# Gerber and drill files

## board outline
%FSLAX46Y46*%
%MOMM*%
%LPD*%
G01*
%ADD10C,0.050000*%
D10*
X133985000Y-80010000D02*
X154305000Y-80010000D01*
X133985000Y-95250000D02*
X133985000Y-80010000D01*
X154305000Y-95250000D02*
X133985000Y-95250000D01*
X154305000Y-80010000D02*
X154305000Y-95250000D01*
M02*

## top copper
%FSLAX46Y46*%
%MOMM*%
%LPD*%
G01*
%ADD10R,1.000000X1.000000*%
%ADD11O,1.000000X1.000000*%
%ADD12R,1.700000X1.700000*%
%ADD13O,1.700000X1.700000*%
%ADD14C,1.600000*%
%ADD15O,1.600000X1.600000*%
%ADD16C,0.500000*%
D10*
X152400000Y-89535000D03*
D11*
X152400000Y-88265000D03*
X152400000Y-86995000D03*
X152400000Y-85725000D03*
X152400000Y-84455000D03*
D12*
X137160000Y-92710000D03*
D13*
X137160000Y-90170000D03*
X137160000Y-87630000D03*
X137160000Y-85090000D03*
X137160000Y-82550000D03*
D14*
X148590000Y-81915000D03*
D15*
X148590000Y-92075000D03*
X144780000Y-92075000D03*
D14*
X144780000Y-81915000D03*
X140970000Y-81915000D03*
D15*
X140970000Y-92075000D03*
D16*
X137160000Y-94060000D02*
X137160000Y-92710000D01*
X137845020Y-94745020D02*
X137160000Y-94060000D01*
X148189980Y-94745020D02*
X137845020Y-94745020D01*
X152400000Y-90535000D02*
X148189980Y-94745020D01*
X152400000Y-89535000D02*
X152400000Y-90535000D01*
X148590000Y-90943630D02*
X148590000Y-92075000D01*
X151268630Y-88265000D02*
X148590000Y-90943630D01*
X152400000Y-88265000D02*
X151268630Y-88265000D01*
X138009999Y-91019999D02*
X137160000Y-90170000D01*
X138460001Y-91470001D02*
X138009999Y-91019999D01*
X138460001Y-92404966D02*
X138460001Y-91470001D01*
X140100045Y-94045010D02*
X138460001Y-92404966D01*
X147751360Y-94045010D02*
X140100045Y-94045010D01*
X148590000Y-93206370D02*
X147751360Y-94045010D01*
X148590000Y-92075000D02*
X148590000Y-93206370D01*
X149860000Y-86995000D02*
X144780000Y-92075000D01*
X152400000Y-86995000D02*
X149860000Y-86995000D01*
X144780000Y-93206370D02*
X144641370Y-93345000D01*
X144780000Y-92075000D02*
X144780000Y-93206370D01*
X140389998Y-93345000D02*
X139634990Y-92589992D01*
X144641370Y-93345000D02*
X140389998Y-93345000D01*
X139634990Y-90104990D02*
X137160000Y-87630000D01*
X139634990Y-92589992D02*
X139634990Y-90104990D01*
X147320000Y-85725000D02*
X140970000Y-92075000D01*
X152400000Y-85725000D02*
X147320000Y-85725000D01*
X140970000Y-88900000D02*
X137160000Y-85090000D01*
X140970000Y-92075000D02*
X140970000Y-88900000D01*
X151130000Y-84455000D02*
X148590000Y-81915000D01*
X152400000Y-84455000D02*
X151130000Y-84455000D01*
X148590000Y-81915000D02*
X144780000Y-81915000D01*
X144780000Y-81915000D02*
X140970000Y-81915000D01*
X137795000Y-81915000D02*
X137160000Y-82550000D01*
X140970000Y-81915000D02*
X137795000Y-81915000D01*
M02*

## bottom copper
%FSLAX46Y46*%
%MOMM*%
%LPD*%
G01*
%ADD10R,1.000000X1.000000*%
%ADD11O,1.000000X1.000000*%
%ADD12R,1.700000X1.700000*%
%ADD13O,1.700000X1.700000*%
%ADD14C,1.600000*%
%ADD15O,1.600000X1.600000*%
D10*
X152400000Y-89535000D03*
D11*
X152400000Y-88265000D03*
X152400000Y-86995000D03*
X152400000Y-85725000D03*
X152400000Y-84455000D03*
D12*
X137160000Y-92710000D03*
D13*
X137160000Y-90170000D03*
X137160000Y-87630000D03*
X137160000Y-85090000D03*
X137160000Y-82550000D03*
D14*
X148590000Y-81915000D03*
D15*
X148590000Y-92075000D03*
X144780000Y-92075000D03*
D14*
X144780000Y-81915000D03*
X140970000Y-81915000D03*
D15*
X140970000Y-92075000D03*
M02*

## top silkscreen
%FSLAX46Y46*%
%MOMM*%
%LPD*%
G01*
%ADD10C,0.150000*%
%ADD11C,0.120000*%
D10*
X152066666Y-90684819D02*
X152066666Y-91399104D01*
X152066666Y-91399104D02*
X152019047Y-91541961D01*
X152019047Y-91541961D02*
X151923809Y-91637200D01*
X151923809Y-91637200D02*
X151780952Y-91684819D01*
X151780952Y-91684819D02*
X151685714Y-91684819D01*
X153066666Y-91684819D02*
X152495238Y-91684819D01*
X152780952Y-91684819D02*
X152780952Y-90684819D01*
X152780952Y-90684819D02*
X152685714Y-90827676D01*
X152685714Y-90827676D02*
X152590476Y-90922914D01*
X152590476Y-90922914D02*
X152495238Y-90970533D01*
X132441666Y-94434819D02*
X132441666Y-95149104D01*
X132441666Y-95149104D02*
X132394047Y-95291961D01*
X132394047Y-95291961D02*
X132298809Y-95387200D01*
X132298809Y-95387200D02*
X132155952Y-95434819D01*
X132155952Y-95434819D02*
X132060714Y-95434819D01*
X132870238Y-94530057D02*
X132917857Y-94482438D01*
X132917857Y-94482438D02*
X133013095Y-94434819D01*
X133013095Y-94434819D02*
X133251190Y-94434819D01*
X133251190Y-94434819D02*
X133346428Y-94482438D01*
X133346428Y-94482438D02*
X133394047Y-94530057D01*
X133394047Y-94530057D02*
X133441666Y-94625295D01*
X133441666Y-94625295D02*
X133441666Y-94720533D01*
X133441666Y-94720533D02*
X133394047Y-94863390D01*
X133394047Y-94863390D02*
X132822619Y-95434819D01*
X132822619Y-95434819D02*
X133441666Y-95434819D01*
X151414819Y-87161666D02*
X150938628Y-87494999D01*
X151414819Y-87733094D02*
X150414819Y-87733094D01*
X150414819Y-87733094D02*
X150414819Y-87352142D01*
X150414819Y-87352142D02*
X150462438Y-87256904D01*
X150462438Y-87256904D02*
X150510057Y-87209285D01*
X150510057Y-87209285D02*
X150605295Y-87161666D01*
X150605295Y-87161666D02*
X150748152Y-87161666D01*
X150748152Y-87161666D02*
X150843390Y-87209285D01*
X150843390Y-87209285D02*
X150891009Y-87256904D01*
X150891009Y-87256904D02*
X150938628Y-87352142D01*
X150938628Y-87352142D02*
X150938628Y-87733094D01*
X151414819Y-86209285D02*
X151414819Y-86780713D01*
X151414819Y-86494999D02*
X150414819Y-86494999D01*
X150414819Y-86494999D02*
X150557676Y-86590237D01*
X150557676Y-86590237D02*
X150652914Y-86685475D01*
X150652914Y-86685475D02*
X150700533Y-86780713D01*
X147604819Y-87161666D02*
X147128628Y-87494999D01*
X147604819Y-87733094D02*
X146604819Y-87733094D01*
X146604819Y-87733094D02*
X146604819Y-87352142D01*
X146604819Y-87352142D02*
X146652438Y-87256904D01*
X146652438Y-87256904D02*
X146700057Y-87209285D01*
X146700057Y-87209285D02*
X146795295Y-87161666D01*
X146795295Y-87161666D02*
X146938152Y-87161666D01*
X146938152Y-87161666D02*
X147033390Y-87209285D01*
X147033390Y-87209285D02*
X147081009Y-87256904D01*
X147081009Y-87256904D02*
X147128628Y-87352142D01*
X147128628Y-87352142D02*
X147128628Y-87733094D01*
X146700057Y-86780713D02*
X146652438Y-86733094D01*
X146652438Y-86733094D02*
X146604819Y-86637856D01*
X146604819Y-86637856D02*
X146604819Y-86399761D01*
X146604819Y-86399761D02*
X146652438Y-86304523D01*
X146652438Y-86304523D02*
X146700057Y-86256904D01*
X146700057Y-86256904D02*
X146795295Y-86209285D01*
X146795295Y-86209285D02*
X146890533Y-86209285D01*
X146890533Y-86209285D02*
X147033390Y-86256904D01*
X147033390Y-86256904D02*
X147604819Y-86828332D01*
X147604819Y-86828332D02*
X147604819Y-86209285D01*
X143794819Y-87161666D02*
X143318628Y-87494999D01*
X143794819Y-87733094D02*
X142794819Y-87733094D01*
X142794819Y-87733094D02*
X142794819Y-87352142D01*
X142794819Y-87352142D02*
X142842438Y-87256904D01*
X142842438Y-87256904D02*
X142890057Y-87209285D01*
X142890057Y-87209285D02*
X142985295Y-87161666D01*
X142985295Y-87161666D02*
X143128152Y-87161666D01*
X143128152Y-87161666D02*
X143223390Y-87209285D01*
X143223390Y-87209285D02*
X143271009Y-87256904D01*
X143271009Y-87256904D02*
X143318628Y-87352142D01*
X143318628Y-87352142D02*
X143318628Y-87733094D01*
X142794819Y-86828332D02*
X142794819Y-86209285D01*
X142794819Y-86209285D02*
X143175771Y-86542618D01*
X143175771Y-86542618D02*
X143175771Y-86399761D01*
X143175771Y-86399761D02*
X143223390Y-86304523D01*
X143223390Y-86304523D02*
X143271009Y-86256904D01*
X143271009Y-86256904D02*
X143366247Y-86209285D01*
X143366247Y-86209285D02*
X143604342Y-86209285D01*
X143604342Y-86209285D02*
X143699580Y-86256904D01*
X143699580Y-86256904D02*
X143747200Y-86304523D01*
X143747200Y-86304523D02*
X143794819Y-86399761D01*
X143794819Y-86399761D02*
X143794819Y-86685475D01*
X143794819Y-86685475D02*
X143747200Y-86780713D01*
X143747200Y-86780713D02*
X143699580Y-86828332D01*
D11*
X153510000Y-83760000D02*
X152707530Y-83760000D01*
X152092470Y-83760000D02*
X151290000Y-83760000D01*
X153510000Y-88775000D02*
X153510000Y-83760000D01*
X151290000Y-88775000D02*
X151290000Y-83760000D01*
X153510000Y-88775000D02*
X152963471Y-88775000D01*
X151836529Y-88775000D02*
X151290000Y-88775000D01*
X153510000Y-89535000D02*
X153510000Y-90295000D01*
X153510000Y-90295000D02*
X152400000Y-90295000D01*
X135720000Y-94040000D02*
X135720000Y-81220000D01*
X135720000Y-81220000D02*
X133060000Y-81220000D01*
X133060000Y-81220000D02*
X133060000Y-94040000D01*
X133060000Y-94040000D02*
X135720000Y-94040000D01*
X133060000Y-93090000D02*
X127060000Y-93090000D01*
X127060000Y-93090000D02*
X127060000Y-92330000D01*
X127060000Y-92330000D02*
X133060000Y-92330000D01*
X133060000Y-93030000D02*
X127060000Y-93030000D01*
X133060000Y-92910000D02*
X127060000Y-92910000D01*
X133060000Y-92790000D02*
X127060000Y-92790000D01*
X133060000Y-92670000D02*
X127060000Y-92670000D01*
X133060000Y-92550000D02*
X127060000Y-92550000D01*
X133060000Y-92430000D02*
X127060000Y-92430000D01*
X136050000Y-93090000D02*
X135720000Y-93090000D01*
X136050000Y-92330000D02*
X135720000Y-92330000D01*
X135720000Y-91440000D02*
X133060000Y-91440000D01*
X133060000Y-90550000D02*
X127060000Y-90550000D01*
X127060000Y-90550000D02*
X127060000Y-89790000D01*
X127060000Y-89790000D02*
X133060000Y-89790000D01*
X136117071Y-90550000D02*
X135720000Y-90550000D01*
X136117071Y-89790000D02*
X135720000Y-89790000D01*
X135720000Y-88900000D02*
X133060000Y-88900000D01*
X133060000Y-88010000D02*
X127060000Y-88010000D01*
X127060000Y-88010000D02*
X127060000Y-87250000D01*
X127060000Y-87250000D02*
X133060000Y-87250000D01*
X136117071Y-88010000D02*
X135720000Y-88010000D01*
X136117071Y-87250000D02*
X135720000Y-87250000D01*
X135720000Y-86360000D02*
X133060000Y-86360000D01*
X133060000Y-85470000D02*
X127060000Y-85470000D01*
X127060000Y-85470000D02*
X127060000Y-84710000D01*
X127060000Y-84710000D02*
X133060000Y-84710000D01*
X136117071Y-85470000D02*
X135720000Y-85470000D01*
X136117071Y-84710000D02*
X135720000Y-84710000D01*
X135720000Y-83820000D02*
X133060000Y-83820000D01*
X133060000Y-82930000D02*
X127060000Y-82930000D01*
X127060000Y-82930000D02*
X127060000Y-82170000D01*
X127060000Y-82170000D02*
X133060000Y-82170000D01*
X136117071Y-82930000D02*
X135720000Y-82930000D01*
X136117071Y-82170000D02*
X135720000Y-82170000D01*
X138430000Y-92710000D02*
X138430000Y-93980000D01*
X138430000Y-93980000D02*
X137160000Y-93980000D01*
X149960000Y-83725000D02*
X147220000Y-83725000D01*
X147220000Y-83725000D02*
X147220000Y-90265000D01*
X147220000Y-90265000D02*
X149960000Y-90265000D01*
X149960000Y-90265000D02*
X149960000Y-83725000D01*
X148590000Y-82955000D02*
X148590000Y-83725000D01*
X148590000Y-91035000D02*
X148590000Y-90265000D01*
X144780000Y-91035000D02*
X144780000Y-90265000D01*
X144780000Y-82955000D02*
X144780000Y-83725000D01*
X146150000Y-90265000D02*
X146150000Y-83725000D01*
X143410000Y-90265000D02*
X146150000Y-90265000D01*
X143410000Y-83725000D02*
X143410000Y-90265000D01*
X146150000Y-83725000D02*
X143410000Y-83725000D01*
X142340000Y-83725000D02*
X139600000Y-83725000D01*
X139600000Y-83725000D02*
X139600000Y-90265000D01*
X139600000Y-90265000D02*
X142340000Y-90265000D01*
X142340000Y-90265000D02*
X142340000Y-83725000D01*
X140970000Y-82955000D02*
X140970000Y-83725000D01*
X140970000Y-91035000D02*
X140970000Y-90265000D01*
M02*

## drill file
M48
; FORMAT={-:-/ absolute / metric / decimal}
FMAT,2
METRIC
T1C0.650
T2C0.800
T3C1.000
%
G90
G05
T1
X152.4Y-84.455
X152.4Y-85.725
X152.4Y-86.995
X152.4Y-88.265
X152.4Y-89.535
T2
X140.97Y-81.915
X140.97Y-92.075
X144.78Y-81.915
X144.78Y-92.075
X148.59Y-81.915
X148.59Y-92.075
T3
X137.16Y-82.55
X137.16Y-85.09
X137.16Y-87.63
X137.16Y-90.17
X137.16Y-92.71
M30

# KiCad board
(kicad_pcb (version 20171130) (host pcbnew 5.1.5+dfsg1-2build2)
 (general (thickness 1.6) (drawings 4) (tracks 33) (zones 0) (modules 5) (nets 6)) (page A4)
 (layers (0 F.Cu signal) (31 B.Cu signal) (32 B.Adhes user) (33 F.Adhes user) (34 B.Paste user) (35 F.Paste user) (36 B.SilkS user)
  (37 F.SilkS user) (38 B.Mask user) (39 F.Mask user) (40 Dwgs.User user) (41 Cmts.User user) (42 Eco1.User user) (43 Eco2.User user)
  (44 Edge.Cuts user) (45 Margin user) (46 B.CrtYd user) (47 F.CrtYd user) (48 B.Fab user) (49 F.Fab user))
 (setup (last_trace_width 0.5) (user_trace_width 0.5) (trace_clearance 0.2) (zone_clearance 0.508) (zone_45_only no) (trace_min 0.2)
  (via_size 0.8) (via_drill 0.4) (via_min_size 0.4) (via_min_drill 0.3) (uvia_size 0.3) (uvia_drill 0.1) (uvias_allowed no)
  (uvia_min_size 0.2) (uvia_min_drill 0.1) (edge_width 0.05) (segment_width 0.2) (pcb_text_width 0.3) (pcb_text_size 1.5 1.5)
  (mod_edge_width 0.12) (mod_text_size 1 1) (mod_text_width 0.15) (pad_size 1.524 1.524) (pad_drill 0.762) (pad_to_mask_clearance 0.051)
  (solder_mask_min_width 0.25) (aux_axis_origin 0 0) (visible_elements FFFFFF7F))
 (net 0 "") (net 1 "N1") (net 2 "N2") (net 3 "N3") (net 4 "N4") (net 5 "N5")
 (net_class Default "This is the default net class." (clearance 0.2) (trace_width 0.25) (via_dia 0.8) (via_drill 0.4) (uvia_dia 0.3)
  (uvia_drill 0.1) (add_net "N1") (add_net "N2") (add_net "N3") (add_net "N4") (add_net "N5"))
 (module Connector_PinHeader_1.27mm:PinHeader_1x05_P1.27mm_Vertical (layer F.Cu) (at 152.4 89.535 180)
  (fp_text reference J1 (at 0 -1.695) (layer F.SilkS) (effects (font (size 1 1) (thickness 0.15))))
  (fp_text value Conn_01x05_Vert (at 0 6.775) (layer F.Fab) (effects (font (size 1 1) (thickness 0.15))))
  (fp_line (start -1.11 5.775) (end -0.30753 5.775) (layer F.SilkS) (width 0.12))
  (fp_line (start 0.30753 5.775) (end 1.11 5.775) (layer F.SilkS) (width 0.12))
  (fp_line (start -1.11 0.76) (end -1.11 5.775) (layer F.SilkS) (width 0.12))
  (fp_line (start 1.11 0.76) (end 1.11 5.775) (layer F.SilkS) (width 0.12))
  (fp_line (start -1.11 0.76) (end -0.563471 0.76) (layer F.SilkS) (width 0.12))
  (fp_line (start 0.563471 0.76) (end 1.11 0.76) (layer F.SilkS) (width 0.12))
  (fp_line (start -1.11 0) (end -1.11 -0.76) (layer F.SilkS) (width 0.12))
  (fp_line (start -1.11 -0.76) (end 0 -0.76) (layer F.SilkS) (width 0.12))
  (pad 1 thru_hole rect (at 0 0 180) (size 1 1) (drill 0.65) (layers *.Cu *.Mask) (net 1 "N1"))
  (pad 2 thru_hole oval (at 0 1.27 180) (size 1 1) (drill 0.65) (layers *.Cu *.Mask) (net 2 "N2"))
  (pad 3 thru_hole oval (at 0 2.54 180) (size 1 1) (drill 0.65) (layers *.Cu *.Mask) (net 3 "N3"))
  (pad 4 thru_hole oval (at 0 3.81 180) (size 1 1) (drill 0.65) (layers *.Cu *.Mask) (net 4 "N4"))
  (pad 5 thru_hole oval (at 0 5.08 180) (size 1 1) (drill 0.65) (layers *.Cu *.Mask) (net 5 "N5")))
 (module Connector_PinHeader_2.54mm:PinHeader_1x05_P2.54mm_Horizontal (layer F.Cu) (at 137.16 92.71 180)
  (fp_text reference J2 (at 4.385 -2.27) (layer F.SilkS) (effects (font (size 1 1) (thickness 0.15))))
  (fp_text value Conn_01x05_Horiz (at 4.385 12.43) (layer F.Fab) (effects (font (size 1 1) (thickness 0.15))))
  (fp_line (start 1.44 -1.33) (end 1.44 11.49) (layer F.SilkS) (width 0.12))
  (fp_line (start 1.44 11.49) (end 4.1 11.49) (layer F.SilkS) (width 0.12))
  (fp_line (start 4.1 11.49) (end 4.1 -1.33) (layer F.SilkS) (width 0.12))
  (fp_line (start 4.1 -1.33) (end 1.44 -1.33) (layer F.SilkS) (width 0.12))
  (fp_line (start 4.1 -0.38) (end 10.1 -0.38) (layer F.SilkS) (width 0.12))
  (fp_line (start 10.1 -0.38) (end 10.1 0.38) (layer F.SilkS) (width 0.12))
  (fp_line (start 10.1 0.38) (end 4.1 0.38) (layer F.SilkS) (width 0.12))
  (fp_line (start 4.1 -0.32) (end 10.1 -0.32) (layer F.SilkS) (width 0.12))
  (fp_line (start 4.1 -0.2) (end 10.1 -0.2) (layer F.SilkS) (width 0.12))
  (fp_line (start 4.1 -0.08) (end 10.1 -0.08) (layer F.SilkS) (width 0.12))
  (fp_line (start 4.1 0.04) (end 10.1 0.04) (layer F.SilkS) (width 0.12))
  (fp_line (start 4.1 0.16) (end 10.1 0.16) (layer F.SilkS) (width 0.12))
  (fp_line (start 4.1 0.28) (end 10.1 0.28) (layer F.SilkS) (width 0.12))
  (fp_line (start 1.11 -0.38) (end 1.44 -0.38) (layer F.SilkS) (width 0.12))
  (fp_line (start 1.11 0.38) (end 1.44 0.38) (layer F.SilkS) (width 0.12))
  (fp_line (start 1.44 1.27) (end 4.1 1.27) (layer F.SilkS) (width 0.12))
  (fp_line (start 4.1 2.16) (end 10.1 2.16) (layer F.SilkS) (width 0.12))
  (fp_line (start 10.1 2.16) (end 10.1 2.92) (layer F.SilkS) (width 0.12))
  (fp_line (start 10.1 2.92) (end 4.1 2.92) (layer F.SilkS) (width 0.12))
  (fp_line (start 1.042929 2.16) (end 1.44 2.16) (layer F.SilkS) (width 0.12))
  (fp_line (start 1.042929 2.92) (end 1.44 2.92) (layer F.SilkS) (width 0.12))
  (fp_line (start 1.44 3.81) (end 4.1 3.81) (layer F.SilkS) (width 0.12))
  (fp_line (start 4.1 4.7) (end 10.1 4.7) (layer F.SilkS) (width 0.12))
  (fp_line (start 10.1 4.7) (end 10.1 5.46) (layer F.SilkS) (width 0.12))
  (fp_line (start 10.1 5.46) (end 4.1 5.46) (layer F.SilkS) (width 0.12))
  (fp_line (start 1.042929 4.7) (end 1.44 4.7) (layer F.SilkS) (width 0.12))
  (fp_line (start 1.042929 5.46) (end 1.44 5.46) (layer F.SilkS) (width 0.12))
  (fp_line (start 1.44 6.35) (end 4.1 6.35) (layer F.SilkS) (width 0.12))
  (fp_line (start 4.1 7.24) (end 10.1 7.24) (layer F.SilkS) (width 0.12))
  (fp_line (start 10.1 7.24) (end 10.1 8) (layer F.SilkS) (width 0.12))
  (fp_line (start 10.1 8) (end 4.1 8) (layer F.SilkS) (width 0.12))
  (fp_line (start 1.042929 7.24) (end 1.44 7.24) (layer F.SilkS) (width 0.12))
  (fp_line (start 1.042929 8) (end 1.44 8) (layer F.SilkS) (width 0.12))
  (fp_line (start 1.44 8.89) (end 4.1 8.89) (layer F.SilkS) (width 0.12))
  (fp_line (start 4.1 9.78) (end 10.1 9.78) (layer F.SilkS) (width 0.12))
  (fp_line (start 10.1 9.78) (end 10.1 10.54) (layer F.SilkS) (width 0.12))
  (fp_line (start 10.1 10.54) (end 4.1 10.54) (layer F.SilkS) (width 0.12))
  (fp_line (start 1.042929 9.78) (end 1.44 9.78) (layer F.SilkS) (width 0.12))
  (fp_line (start 1.042929 10.54) (end 1.44 10.54) (layer F.SilkS) (width 0.12))
  (fp_line (start -1.27 0) (end -1.27 -1.27) (layer F.SilkS) (width 0.12))
  (fp_line (start -1.27 -1.27) (end 0 -1.27) (layer F.SilkS) (width 0.12))
  (pad 1 thru_hole rect (at 0 0 180) (size 1.7 1.7) (drill 1) (layers *.Cu *.Mask) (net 1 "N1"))
  (pad 2 thru_hole oval (at 0 2.54 180) (size 1.7 1.7) (drill 1) (layers *.Cu *.Mask) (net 2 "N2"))
  (pad 3 thru_hole oval (at 0 5.08 180) (size 1.7 1.7) (drill 1) (layers *.Cu *.Mask) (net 3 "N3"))
  (pad 4 thru_hole oval (at 0 7.62 180) (size 1.7 1.7) (drill 1) (layers *.Cu *.Mask) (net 4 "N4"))
  (pad 5 thru_hole oval (at 0 10.16 180) (size 1.7 1.7) (drill 1) (layers *.Cu *.Mask) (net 5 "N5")))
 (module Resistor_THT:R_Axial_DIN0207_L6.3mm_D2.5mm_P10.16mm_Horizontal (layer F.Cu) (at 148.59 81.915 270)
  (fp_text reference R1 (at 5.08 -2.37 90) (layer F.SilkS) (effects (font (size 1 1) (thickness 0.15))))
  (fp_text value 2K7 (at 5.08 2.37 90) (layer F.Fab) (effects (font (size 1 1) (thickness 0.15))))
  (fp_line (start 1.81 -1.37) (end 1.81 1.37) (layer F.SilkS) (width 0.12))
  (fp_line (start 1.81 1.37) (end 8.35 1.37) (layer F.SilkS) (width 0.12))
  (fp_line (start 8.35 1.37) (end 8.35 -1.37) (layer F.SilkS) (width 0.12))
  (fp_line (start 8.35 -1.37) (end 1.81 -1.37) (layer F.SilkS) (width 0.12))
  (fp_line (start 1.04 0) (end 1.81 0) (layer F.SilkS) (width 0.12))
  (fp_line (start 9.12 0) (end 8.35 0) (layer F.SilkS) (width 0.12))
  (pad 1 thru_hole circle (at 0 0 270) (size 1.6 1.6) (drill 0.8) (layers *.Cu *.Mask) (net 5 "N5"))
  (pad 2 thru_hole oval (at 10.16 0 270) (size 1.6 1.6) (drill 0.8) (layers *.Cu *.Mask) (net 2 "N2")))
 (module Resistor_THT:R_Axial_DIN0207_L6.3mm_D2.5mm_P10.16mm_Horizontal (layer F.Cu) (at 144.78 81.915 270)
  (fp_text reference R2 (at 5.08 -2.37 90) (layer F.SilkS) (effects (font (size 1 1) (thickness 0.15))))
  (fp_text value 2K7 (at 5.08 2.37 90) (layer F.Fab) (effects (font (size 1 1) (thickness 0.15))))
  (fp_line (start 9.12 0) (end 8.35 0) (layer F.SilkS) (width 0.12))
  (fp_line (start 1.04 0) (end 1.81 0) (layer F.SilkS) (width 0.12))
  (fp_line (start 8.35 -1.37) (end 1.81 -1.37) (layer F.SilkS) (width 0.12))
  (fp_line (start 8.35 1.37) (end 8.35 -1.37) (layer F.SilkS) (width 0.12))
  (fp_line (start 1.81 1.37) (end 8.35 1.37) (layer F.SilkS) (width 0.12))
  (fp_line (start 1.81 -1.37) (end 1.81 1.37) (layer F.SilkS) (width 0.12))
  (pad 2 thru_hole oval (at 10.16 0 270) (size 1.6 1.6) (drill 0.8) (layers *.Cu *.Mask) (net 3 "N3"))
  (pad 1 thru_hole circle (at 0 0 270) (size 1.6 1.6) (drill 0.8) (layers *.Cu *.Mask) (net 5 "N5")))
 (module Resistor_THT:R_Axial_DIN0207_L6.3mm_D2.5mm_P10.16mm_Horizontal (layer F.Cu) (at 140.97 81.915 270)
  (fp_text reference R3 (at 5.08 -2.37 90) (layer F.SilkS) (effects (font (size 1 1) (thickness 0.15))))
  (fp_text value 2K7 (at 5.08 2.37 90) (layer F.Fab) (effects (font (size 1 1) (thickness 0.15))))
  (fp_line (start 1.81 -1.37) (end 1.81 1.37) (layer F.SilkS) (width 0.12))
  (fp_line (start 1.81 1.37) (end 8.35 1.37) (layer F.SilkS) (width 0.12))
  (fp_line (start 8.35 1.37) (end 8.35 -1.37) (layer F.SilkS) (width 0.12))
  (fp_line (start 8.35 -1.37) (end 1.81 -1.37) (layer F.SilkS) (width 0.12))
  (fp_line (start 1.04 0) (end 1.81 0) (layer F.SilkS) (width 0.12))
  (fp_line (start 9.12 0) (end 8.35 0) (layer F.SilkS) (width 0.12))
  (pad 1 thru_hole circle (at 0 0 270) (size 1.6 1.6) (drill 0.8) (layers *.Cu *.Mask) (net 5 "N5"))
  (pad 2 thru_hole oval (at 10.16 0 270) (size 1.6 1.6) (drill 0.8) (layers *.Cu *.Mask) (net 4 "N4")))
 (gr_line (start 133.985 80.01) (end 154.305 80.01) (layer Edge.Cuts) (width 0.05))
 (gr_line (start 133.985 95.25) (end 133.985 80.01) (layer Edge.Cuts) (width 0.05))
 (gr_line (start 154.305 95.25) (end 133.985 95.25) (layer Edge.Cuts) (width 0.05))
 (gr_line (start 154.305 80.01) (end 154.305 95.25) (layer Edge.Cuts) (width 0.05))
 (segment (start 137.16 94.06) (end 137.16 92.71) (width 0.5) (layer F.Cu) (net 1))
 (segment (start 137.84502 94.74502) (end 137.16 94.06) (width 0.5) (layer F.Cu) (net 1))
 (segment (start 148.18998 94.74502) (end 137.84502 94.74502) (width 0.5) (layer F.Cu) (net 1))
 (segment (start 152.4 90.535) (end 148.18998 94.74502) (width 0.5) (layer F.Cu) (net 1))
 (segment (start 152.4 89.535) (end 152.4 90.535) (width 0.5) (layer F.Cu) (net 1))
 (segment (start 148.59 90.94363) (end 148.59 92.075) (width 0.5) (layer F.Cu) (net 2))
 (segment (start 151.26863 88.265) (end 148.59 90.94363) (width 0.5) (layer F.Cu) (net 2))
 (segment (start 152.4 88.265) (end 151.26863 88.265) (width 0.5) (layer F.Cu) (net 2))
 (segment (start 138.009999 91.019999) (end 137.16 90.17) (width 0.5) (layer F.Cu) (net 2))
 (segment (start 138.460001 91.470001) (end 138.009999 91.019999) (width 0.5) (layer F.Cu) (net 2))
 (segment (start 138.460001 92.404966) (end 138.460001 91.470001) (width 0.5) (layer F.Cu) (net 2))
 (segment (start 140.100045 94.04501) (end 138.460001 92.404966) (width 0.5) (layer F.Cu) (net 2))
 (segment (start 147.75136 94.04501) (end 140.100045 94.04501) (width 0.5) (layer F.Cu) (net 2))
 (segment (start 148.59 93.20637) (end 147.75136 94.04501) (width 0.5) (layer F.Cu) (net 2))
 (segment (start 148.59 92.075) (end 148.59 93.20637) (width 0.5) (layer F.Cu) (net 2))
 (segment (start 149.86 86.995) (end 144.78 92.075) (width 0.5) (layer F.Cu) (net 3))
 (segment (start 152.4 86.995) (end 149.86 86.995) (width 0.5) (layer F.Cu) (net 3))
 (segment (start 144.78 93.20637) (end 144.64137 93.345) (width 0.5) (layer F.Cu) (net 3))
 (segment (start 144.78 92.075) (end 144.78 93.20637) (width 0.5) (layer F.Cu) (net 3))
 (segment (start 140.389998 93.345) (end 139.63499 92.589992) (width 0.5) (layer F.Cu) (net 3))
 (segment (start 144.64137 93.345) (end 140.389998 93.345) (width 0.5) (layer F.Cu) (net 3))
 (segment (start 139.63499 90.10499) (end 137.16 87.63) (width 0.5) (layer F.Cu) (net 3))
 (segment (start 139.63499 92.589992) (end 139.63499 90.10499) (width 0.5) (layer F.Cu) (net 3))
 (segment (start 147.32 85.725) (end 140.97 92.075) (width 0.5) (layer F.Cu) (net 4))
 (segment (start 152.4 85.725) (end 147.32 85.725) (width 0.5) (layer F.Cu) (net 4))
 (segment (start 140.97 88.9) (end 137.16 85.09) (width 0.5) (layer F.Cu) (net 4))
 (segment (start 140.97 92.075) (end 140.97 88.9) (width 0.5) (layer F.Cu) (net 4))
 (segment (start 151.13 84.455) (end 148.59 81.915) (width 0.5) (layer F.Cu) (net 5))
 (segment (start 152.4 84.455) (end 151.13 84.455) (width 0.5) (layer F.Cu) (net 5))
 (segment (start 148.59 81.915) (end 144.78 81.915) (width 0.5) (layer F.Cu) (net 5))
 (segment (start 144.78 81.915) (end 140.97 81.915) (width 0.5) (layer F.Cu) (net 5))
 (segment (start 137.795 81.915) (end 137.16 82.55) (width 0.5) (layer F.Cu) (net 5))
 (segment (start 140.97 81.915) (end 137.795 81.915) (width 0.5) (layer F.Cu) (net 5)))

